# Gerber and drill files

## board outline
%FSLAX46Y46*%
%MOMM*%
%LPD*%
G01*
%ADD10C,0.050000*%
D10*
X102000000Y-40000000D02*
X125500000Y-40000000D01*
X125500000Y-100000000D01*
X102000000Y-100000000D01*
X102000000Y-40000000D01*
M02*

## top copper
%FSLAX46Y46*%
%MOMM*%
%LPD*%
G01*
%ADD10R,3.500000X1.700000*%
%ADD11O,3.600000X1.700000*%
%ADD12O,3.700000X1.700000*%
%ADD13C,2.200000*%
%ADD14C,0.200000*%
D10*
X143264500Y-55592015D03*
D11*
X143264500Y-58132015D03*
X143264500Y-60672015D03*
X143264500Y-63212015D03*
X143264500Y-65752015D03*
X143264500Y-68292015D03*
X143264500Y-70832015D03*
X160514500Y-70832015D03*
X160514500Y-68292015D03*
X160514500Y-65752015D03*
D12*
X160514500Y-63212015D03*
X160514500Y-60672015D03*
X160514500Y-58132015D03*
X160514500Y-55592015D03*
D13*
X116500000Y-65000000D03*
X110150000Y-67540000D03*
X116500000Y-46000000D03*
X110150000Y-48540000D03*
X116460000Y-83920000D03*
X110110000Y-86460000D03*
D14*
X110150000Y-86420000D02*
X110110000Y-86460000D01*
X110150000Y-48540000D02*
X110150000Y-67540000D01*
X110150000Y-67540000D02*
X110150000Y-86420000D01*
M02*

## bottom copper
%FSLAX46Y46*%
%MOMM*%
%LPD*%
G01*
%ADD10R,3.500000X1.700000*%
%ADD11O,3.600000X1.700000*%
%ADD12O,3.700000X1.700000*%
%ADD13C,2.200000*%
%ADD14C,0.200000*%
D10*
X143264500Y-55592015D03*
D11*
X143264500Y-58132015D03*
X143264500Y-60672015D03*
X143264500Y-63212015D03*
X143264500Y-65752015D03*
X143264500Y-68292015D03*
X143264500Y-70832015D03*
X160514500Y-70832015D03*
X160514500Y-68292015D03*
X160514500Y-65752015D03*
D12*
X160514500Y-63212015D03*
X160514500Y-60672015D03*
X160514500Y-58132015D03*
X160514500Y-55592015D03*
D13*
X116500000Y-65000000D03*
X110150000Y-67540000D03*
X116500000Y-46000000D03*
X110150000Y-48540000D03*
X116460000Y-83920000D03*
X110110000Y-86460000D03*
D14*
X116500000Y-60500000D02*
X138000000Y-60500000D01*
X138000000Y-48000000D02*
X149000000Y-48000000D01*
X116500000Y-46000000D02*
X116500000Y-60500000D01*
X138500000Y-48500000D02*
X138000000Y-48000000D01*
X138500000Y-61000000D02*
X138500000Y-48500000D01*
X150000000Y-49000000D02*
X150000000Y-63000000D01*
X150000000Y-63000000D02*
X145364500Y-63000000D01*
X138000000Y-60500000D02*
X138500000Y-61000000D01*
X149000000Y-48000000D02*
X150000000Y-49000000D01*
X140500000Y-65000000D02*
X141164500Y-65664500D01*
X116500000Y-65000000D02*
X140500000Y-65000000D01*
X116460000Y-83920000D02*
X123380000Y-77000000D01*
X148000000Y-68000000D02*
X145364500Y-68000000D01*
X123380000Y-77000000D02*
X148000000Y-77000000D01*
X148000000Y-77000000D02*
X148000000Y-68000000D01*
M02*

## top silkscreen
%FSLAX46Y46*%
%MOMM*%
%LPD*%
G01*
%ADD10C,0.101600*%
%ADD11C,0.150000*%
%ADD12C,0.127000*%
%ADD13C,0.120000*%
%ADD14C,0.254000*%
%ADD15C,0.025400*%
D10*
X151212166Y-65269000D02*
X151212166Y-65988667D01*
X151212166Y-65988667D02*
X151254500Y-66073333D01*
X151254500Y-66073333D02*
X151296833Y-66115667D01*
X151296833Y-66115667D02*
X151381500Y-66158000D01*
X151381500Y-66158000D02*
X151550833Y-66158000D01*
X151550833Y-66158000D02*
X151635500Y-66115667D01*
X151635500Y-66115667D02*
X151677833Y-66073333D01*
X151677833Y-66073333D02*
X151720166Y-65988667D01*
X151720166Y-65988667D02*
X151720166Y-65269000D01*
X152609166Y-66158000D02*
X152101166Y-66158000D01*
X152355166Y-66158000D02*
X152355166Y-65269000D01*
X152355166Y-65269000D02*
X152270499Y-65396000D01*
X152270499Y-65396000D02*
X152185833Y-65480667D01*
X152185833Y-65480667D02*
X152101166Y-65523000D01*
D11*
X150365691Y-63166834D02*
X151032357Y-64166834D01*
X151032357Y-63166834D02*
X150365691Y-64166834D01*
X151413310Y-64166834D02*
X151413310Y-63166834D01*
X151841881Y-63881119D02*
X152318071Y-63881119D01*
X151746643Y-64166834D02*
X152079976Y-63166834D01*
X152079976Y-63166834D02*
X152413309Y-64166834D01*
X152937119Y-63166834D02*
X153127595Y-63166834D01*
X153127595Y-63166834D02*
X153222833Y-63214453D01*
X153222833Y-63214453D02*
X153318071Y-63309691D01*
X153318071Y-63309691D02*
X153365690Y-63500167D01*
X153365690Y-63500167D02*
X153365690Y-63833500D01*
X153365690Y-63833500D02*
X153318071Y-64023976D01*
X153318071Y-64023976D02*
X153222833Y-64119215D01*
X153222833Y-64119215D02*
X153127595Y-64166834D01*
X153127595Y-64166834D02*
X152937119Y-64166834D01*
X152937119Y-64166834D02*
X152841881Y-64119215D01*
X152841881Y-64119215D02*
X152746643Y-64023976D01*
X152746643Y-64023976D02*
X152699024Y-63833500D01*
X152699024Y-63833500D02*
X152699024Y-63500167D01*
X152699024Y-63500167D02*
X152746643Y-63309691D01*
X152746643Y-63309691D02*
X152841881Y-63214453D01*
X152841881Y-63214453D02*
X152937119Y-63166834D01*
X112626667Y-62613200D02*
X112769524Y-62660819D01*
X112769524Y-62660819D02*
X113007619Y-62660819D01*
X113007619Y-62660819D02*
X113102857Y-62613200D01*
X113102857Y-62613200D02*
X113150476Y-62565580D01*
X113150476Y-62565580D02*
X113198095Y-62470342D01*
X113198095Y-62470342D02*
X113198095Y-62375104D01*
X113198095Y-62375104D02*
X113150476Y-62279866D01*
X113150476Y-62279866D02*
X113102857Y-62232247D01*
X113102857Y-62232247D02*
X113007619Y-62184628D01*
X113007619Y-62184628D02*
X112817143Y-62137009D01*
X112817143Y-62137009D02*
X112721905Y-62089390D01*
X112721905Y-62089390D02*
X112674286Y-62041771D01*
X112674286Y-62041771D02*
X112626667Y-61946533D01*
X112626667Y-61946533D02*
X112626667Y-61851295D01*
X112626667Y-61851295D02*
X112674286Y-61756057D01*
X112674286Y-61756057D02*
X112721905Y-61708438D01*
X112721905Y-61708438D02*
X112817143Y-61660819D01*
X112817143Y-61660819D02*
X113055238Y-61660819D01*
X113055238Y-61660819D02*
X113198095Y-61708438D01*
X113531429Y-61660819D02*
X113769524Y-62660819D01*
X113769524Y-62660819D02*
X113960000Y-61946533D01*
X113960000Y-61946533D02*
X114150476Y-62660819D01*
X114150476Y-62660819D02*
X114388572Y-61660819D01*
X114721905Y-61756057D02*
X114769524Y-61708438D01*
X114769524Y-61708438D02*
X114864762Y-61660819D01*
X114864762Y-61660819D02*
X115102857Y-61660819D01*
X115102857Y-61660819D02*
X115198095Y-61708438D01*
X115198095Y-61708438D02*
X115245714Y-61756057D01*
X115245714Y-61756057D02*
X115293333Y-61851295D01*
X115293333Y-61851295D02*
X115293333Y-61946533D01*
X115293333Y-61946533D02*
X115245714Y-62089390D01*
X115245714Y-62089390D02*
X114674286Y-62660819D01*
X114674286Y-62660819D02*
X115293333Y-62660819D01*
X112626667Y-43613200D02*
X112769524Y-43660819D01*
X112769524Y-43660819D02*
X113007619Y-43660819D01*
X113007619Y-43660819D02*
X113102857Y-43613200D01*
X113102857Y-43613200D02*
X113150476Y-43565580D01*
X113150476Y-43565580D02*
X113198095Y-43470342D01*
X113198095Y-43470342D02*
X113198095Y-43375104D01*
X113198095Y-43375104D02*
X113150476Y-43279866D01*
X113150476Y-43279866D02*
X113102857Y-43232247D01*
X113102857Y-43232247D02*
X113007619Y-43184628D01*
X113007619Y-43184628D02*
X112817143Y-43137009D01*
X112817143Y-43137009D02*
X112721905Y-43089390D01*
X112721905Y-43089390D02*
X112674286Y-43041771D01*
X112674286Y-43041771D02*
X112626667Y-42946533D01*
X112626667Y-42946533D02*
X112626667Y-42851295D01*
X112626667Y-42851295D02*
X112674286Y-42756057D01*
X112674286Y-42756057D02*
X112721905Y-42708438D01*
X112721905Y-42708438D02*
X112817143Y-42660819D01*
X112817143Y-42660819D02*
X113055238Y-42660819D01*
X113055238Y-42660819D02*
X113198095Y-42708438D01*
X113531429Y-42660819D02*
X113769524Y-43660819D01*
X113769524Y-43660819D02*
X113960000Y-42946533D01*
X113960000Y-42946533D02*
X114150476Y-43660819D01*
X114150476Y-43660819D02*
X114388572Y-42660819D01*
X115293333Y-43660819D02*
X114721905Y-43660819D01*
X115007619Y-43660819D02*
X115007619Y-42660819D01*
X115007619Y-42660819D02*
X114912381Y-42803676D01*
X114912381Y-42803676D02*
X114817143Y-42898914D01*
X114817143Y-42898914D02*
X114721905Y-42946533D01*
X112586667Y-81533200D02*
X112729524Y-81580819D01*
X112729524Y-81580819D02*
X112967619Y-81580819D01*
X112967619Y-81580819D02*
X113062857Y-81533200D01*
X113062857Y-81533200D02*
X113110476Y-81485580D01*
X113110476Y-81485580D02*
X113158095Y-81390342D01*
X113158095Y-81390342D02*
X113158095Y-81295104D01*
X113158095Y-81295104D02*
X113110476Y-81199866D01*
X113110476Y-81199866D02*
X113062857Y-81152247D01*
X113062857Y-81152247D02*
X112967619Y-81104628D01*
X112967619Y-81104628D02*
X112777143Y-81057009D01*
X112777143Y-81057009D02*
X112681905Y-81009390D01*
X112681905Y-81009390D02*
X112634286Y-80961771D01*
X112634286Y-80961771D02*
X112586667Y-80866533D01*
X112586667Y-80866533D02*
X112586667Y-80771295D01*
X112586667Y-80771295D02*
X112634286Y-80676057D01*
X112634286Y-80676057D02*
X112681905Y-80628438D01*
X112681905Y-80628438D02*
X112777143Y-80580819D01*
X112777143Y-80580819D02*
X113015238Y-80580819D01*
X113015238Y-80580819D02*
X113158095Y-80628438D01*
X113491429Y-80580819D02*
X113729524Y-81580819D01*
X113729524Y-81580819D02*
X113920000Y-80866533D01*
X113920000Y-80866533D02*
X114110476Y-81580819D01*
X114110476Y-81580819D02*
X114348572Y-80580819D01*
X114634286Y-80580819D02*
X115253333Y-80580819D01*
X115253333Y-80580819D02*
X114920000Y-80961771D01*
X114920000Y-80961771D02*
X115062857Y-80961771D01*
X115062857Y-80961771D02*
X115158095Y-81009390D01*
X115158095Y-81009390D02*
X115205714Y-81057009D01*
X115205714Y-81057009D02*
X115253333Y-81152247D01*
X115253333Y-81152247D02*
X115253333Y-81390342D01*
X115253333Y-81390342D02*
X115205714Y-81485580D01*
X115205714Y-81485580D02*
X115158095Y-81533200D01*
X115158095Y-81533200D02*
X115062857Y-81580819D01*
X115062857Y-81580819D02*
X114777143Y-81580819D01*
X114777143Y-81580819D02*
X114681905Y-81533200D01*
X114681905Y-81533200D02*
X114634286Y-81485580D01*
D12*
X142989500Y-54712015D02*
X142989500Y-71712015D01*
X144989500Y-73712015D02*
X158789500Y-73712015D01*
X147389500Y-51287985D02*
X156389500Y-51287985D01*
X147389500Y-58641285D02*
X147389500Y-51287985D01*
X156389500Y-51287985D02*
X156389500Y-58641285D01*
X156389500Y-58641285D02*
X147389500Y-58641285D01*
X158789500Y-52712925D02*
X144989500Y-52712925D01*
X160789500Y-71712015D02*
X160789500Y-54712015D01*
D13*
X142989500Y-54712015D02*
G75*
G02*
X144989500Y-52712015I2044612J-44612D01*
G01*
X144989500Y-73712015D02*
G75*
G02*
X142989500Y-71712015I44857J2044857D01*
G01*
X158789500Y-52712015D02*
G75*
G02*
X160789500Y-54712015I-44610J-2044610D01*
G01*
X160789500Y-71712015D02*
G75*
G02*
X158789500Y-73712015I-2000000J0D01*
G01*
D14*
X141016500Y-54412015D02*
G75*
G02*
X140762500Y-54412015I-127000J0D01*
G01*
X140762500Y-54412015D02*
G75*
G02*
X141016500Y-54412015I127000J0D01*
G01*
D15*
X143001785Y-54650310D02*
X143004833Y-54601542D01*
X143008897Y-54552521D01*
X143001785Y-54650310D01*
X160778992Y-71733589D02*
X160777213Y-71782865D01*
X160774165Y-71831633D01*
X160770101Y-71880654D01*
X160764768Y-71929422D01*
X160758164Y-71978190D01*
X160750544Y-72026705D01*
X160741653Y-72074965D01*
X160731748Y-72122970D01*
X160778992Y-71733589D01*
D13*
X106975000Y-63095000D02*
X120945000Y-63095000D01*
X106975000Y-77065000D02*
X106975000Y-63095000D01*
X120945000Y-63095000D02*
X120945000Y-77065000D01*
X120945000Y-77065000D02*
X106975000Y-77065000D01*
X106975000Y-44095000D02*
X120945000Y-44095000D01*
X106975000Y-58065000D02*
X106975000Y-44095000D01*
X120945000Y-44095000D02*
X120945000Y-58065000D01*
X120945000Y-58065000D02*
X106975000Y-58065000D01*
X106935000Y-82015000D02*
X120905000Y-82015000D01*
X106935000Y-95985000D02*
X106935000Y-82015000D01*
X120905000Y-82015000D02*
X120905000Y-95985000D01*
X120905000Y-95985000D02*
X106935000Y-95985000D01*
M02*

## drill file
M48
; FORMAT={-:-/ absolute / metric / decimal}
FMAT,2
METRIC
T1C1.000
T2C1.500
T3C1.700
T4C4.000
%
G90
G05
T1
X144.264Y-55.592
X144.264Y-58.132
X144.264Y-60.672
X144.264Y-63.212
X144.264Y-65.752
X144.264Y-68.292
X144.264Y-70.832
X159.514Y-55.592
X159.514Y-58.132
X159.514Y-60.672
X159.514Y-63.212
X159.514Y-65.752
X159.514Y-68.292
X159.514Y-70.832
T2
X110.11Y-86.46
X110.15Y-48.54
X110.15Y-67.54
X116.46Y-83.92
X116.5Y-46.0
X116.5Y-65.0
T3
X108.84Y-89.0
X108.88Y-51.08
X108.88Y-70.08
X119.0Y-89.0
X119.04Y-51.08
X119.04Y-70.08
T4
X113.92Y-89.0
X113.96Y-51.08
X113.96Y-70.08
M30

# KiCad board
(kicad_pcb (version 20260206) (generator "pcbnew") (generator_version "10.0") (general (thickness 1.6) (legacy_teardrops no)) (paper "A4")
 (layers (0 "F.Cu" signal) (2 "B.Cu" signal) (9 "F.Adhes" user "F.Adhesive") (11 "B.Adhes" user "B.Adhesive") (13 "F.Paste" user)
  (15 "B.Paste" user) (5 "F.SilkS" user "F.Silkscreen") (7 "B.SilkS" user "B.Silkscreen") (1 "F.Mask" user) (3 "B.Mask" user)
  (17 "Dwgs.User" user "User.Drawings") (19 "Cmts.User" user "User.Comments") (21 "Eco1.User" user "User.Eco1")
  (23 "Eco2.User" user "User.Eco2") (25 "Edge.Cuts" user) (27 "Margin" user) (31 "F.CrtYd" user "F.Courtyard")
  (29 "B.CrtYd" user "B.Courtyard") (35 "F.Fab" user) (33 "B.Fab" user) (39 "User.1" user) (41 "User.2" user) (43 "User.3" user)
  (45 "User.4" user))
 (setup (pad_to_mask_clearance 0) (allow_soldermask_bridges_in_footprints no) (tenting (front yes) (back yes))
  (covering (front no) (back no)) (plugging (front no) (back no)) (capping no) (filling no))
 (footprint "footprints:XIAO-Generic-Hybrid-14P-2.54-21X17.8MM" (layer "F.Cu") (at 151.8895 63.212015)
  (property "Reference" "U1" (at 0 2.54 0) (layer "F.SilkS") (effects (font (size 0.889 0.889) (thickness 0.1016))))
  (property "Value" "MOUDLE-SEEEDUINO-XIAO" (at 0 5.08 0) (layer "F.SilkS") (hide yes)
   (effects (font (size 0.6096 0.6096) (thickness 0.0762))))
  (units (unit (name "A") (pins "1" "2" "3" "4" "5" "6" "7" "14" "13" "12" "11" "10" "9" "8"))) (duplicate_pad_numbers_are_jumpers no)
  (fp_line (start -8.9 -8.5) (end -8.9 8.5) (stroke (width 0.127) (type solid)) (layer "F.SilkS"))
  (fp_line (start -6.9 10.5) (end 6.9 10.5) (stroke (width 0.127) (type solid)) (layer "F.SilkS"))
  (fp_line (start -4.5 -11.92403) (end 4.5 -11.92403) (stroke (width 0.127) (type solid)) (layer "F.SilkS"))
  (fp_line (start -4.5 -4.57073) (end -4.5 -11.92403) (stroke (width 0.127) (type solid)) (layer "F.SilkS"))
  (fp_line (start 4.5 -11.92403) (end 4.5 -4.57073) (stroke (width 0.127) (type solid)) (layer "F.SilkS"))
  (fp_line (start 4.5 -4.57073) (end -4.5 -4.57073) (stroke (width 0.127) (type solid)) (layer "F.SilkS"))
  (fp_line (start 6.9 -10.49909) (end -6.9 -10.49909) (stroke (width 0.127) (type solid)) (layer "F.SilkS"))
  (fp_line (start 8.9 8.5) (end 8.9 -8.5) (stroke (width 0.127) (type solid)) (layer "F.SilkS"))
  (fp_arc (start -8.9 -8.5) (mid -8.301491 -9.901491) (end -6.9 -10.5) (stroke (width 0.12) (type solid)) (layer "F.SilkS"))
  (fp_arc (start -6.9 10.5) (mid -8.301423 9.901423) (end -8.9 8.5) (stroke (width 0.12) (type solid)) (layer "F.SilkS"))
  (fp_arc (start 6.9 -10.5) (mid 8.301491 -9.901491) (end 8.9 -8.5) (stroke (width 0.12) (type solid)) (layer "F.SilkS"))
  (fp_arc (start 8.9 8.5) (mid 8.314214 9.914214) (end 6.9 10.5) (stroke (width 0.12) (type solid)) (layer "F.SilkS"))
  (fp_circle (center -11 -8.8) (end -11 -9.054) (stroke (width 0) (type solid)) (fill yes) (layer "F.SilkS"))
  (fp_poly
   (pts (xy -8.887715 -8.561705) (xy -8.884667 -8.610473) (xy -8.880603 -8.659494)) (stroke (width 0.0254) (type solid)) (fill no)
   (layer "F.SilkS"))
  (fp_poly
   (pts (xy 8.889492 8.521574) (xy 8.887713 8.57085) (xy 8.884665 8.619618) (xy 8.880601 8.668639) (xy 8.875268 8.717407)
    (xy 8.868664 8.766175) (xy 8.861044 8.81469) (xy 8.852153 8.86295) (xy 8.842248 8.910955))
   (stroke (width 0.0254) (type solid)) (fill no) (layer "F.SilkS"))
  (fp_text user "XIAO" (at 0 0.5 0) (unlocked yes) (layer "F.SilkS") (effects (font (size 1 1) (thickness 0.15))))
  (pad "1" thru_hole rect (at -7.625 -7.62) (size 3.5 1.7) (drill 1 (offset -1 0)) (layers "*.Cu" "*.Mask") (remove_unused_layers no)
   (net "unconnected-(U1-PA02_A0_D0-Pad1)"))
  (pad "2" thru_hole oval (at -7.625 -5.08) (size 3.6 1.7) (drill 1 (offset -1 0)) (layers "*.Cu" "*.Mask") (remove_unused_layers no)
   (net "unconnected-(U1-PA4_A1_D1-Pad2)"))
  (pad "3" thru_hole oval (at -7.625 -2.54) (size 3.6 1.7) (drill 1 (offset -1 0)) (layers "*.Cu" "*.Mask") (remove_unused_layers no)
   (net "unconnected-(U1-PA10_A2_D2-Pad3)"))
  (pad "4" thru_hole oval (at -7.625 0) (size 3.6 1.7) (drill 1 (offset -1 0)) (layers "*.Cu" "*.Mask") (remove_unused_layers no)
   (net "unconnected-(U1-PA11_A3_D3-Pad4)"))
  (pad "5" thru_hole oval (at -7.625 2.54) (size 3.6 1.7) (drill 1 (offset -1 0)) (layers "*.Cu" "*.Mask") (remove_unused_layers no)
   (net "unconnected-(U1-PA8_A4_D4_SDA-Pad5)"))
  (pad "6" thru_hole oval (at -7.625 5.08 180) (size 3.6 1.7) (drill 1 (offset 1 0)) (layers "*.Cu" "*.Mask") (remove_unused_layers no)
   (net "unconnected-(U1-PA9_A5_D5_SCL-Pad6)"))
  (pad "7" thru_hole oval (at -7.625 7.62) (size 3.6 1.7) (drill 1 (offset -1 0)) (layers "*.Cu" "*.Mask") (remove_unused_layers no)
   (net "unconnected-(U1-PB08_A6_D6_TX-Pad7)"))
  (pad "8" thru_hole oval (at 7.625 7.62) (size 3.6 1.7) (drill 1 (offset 1 0)) (layers "*.Cu" "*.Mask") (remove_unused_layers no)
   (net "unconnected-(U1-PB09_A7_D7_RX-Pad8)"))
  (pad "9" thru_hole oval (at 7.625 5.08) (size 3.6 1.7) (drill 1 (offset 1 0)) (layers "*.Cu" "*.Mask") (remove_unused_layers no)
   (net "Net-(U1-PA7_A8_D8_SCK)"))
  (pad "10" thru_hole oval (at 7.625 2.54) (size 3.6 1.7) (drill 1 (offset 1 0)) (layers "*.Cu" "*.Mask") (remove_unused_layers no)
   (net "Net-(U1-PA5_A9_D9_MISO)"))
  (pad "11" thru_hole oval (at 7.625 0) (size 3.7 1.7) (drill 1 (offset 1 0)) (layers "*.Cu" "*.Mask") (remove_unused_layers no)
   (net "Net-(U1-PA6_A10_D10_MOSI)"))
  (pad "12" thru_hole oval (at 7.625 -2.54) (size 3.7 1.7) (drill 1 (offset 1 0)) (layers "*.Cu" "*.Mask") (remove_unused_layers no)
   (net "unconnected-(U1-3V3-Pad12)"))
  (pad "13" thru_hole oval (at 7.625 -5.08) (size 3.7 1.7) (drill 1 (offset 1 0)) (layers "*.Cu" "*.Mask") (remove_unused_layers no)
   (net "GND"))
  (pad "14" thru_hole oval (at 7.625 -7.62) (size 3.7 1.7) (drill 1 (offset 1 0)) (layers "*.Cu" "*.Mask") (remove_unused_layers no)
   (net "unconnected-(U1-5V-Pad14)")))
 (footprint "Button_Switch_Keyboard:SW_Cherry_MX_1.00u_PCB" (layer "F.Cu") (at 116.5 65)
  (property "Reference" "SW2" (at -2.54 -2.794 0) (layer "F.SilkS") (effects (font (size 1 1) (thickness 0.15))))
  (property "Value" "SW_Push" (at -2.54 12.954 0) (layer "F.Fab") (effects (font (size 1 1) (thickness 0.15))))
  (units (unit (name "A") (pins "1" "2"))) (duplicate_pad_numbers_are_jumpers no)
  (fp_line (start -9.525 -1.905) (end 4.445 -1.905) (stroke (width 0.12) (type solid)) (layer "F.SilkS"))
  (fp_line (start -9.525 12.065) (end -9.525 -1.905) (stroke (width 0.12) (type solid)) (layer "F.SilkS"))
  (fp_line (start 4.445 -1.905) (end 4.445 12.065) (stroke (width 0.12) (type solid)) (layer "F.SilkS"))
  (fp_line (start 4.445 12.065) (end -9.525 12.065) (stroke (width 0.12) (type solid)) (layer "F.SilkS"))
  (pad "" np_thru_hole circle (at -7.62 5.08) (size 1.7 1.7) (drill 1.7) (layers "*.Cu" "*.Mask"))
  (pad "" np_thru_hole circle (at -2.54 5.08) (size 4 4) (drill 4) (layers "*.Cu" "*.Mask"))
  (pad "" np_thru_hole circle (at 2.54 5.08) (size 1.7 1.7) (drill 1.7) (layers "*.Cu" "*.Mask"))
  (pad "1" thru_hole circle (at 0 0) (size 2.2 2.2) (drill 1.5) (layers "*.Cu" "*.Mask") (remove_unused_layers no)
   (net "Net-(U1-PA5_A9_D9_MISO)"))
  (pad "2" thru_hole circle (at -6.35 2.54) (size 2.2 2.2) (drill 1.5) (layers "*.Cu" "*.Mask") (remove_unused_layers no) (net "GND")))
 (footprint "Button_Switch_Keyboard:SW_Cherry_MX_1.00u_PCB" (layer "F.Cu") (at 116.5 46)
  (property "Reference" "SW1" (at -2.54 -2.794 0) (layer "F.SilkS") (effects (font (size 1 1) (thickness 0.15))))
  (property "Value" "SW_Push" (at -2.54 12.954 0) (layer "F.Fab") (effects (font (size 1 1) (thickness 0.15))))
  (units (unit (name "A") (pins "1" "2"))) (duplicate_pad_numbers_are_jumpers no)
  (fp_line (start -9.525 -1.905) (end 4.445 -1.905) (stroke (width 0.12) (type solid)) (layer "F.SilkS"))
  (fp_line (start -9.525 12.065) (end -9.525 -1.905) (stroke (width 0.12) (type solid)) (layer "F.SilkS"))
  (fp_line (start 4.445 -1.905) (end 4.445 12.065) (stroke (width 0.12) (type solid)) (layer "F.SilkS"))
  (fp_line (start 4.445 12.065) (end -9.525 12.065) (stroke (width 0.12) (type solid)) (layer "F.SilkS"))
  (pad "" np_thru_hole circle (at -7.62 5.08) (size 1.7 1.7) (drill 1.7) (layers "*.Cu" "*.Mask"))
  (pad "" np_thru_hole circle (at -2.54 5.08) (size 4 4) (drill 4) (layers "*.Cu" "*.Mask"))
  (pad "" np_thru_hole circle (at 2.54 5.08) (size 1.7 1.7) (drill 1.7) (layers "*.Cu" "*.Mask"))
  (pad "1" thru_hole circle (at 0 0) (size 2.2 2.2) (drill 1.5) (layers "*.Cu" "*.Mask") (remove_unused_layers no)
   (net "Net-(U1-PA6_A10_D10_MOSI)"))
  (pad "2" thru_hole circle (at -6.35 2.54) (size 2.2 2.2) (drill 1.5) (layers "*.Cu" "*.Mask") (remove_unused_layers no) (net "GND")))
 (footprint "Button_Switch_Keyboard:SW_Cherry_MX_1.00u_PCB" (layer "F.Cu") (at 116.46 83.92)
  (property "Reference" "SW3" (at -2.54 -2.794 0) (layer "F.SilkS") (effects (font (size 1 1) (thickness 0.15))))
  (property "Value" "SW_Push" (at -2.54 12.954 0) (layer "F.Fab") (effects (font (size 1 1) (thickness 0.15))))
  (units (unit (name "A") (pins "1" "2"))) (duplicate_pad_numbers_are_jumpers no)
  (fp_line (start -9.525 -1.905) (end 4.445 -1.905) (stroke (width 0.12) (type solid)) (layer "F.SilkS"))
  (fp_line (start -9.525 12.065) (end -9.525 -1.905) (stroke (width 0.12) (type solid)) (layer "F.SilkS"))
  (fp_line (start 4.445 -1.905) (end 4.445 12.065) (stroke (width 0.12) (type solid)) (layer "F.SilkS"))
  (fp_line (start 4.445 12.065) (end -9.525 12.065) (stroke (width 0.12) (type solid)) (layer "F.SilkS"))
  (pad "" np_thru_hole circle (at -7.62 5.08) (size 1.7 1.7) (drill 1.7) (layers "*.Cu" "*.Mask"))
  (pad "" np_thru_hole circle (at -2.54 5.08) (size 4 4) (drill 4) (layers "*.Cu" "*.Mask"))
  (pad "" np_thru_hole circle (at 2.54 5.08) (size 1.7 1.7) (drill 1.7) (layers "*.Cu" "*.Mask"))
  (pad "1" thru_hole circle (at 0 0) (size 2.2 2.2) (drill 1.5) (layers "*.Cu" "*.Mask") (remove_unused_layers no)
   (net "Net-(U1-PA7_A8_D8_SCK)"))
  (pad "2" thru_hole circle (at -6.35 2.54) (size 2.2 2.2) (drill 1.5) (layers "*.Cu" "*.Mask") (remove_unused_layers no) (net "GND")))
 (gr_rect (start 102 40) (end 125.5 100) (stroke (width 0.05) (type default)) (fill no) (layer "Edge.Cuts"))
 (segment (start 116.5 60.5) (end 138 60.5) (width 0.2) (layer "B.Cu") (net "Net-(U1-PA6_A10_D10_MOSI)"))
 (segment (start 138 48) (end 149 48) (width 0.2) (layer "B.Cu") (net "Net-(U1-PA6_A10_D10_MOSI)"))
 (segment (start 116.5 46) (end 116.5 60.5) (width 0.2) (layer "B.Cu") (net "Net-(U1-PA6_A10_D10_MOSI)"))
 (segment (start 138.5 48.5) (end 138 48) (width 0.2) (layer "B.Cu") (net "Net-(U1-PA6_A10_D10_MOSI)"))
 (segment (start 138.5 61) (end 138.5 48.5) (width 0.2) (layer "B.Cu") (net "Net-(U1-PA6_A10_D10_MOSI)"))
 (segment (start 150 49) (end 150 63) (width 0.2) (layer "B.Cu") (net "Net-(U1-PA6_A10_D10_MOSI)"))
 (segment (start 150 63) (end 145.3645 63) (width 0.2) (layer "B.Cu") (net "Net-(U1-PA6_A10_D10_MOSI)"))
 (segment (start 138 60.5) (end 138.5 61) (width 0.2) (layer "B.Cu") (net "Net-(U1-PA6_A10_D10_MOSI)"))
 (segment (start 149 48) (end 150 49) (width 0.2) (layer "B.Cu") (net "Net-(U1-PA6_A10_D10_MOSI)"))
 (segment (start 110.15 86.42) (end 110.11 86.46) (width 0.2) (layer "F.Cu") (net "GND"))
 (segment (start 110.15 48.54) (end 110.15 67.54) (width 0.2) (layer "F.Cu") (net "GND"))
 (segment (start 110.15 67.54) (end 110.15 86.42) (width 0.2) (layer "F.Cu") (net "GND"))
 (segment (start 140.5 65) (end 141.1645 65.6645) (width 0.2) (layer "B.Cu") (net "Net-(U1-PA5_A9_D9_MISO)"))
 (segment (start 116.5 65) (end 140.5 65) (width 0.2) (layer "B.Cu") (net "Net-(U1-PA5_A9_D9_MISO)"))
 (segment (start 116.46 83.92) (end 123.38 77) (width 0.2) (layer "B.Cu") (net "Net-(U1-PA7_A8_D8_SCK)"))
 (segment (start 148 68) (end 145.3645 68) (width 0.2) (layer "B.Cu") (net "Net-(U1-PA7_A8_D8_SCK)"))
 (segment (start 123.38 77) (end 148 77) (width 0.2) (layer "B.Cu") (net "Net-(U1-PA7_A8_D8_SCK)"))
 (segment (start 148 77) (end 148 68) (width 0.2) (layer "B.Cu") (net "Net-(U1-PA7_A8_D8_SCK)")))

